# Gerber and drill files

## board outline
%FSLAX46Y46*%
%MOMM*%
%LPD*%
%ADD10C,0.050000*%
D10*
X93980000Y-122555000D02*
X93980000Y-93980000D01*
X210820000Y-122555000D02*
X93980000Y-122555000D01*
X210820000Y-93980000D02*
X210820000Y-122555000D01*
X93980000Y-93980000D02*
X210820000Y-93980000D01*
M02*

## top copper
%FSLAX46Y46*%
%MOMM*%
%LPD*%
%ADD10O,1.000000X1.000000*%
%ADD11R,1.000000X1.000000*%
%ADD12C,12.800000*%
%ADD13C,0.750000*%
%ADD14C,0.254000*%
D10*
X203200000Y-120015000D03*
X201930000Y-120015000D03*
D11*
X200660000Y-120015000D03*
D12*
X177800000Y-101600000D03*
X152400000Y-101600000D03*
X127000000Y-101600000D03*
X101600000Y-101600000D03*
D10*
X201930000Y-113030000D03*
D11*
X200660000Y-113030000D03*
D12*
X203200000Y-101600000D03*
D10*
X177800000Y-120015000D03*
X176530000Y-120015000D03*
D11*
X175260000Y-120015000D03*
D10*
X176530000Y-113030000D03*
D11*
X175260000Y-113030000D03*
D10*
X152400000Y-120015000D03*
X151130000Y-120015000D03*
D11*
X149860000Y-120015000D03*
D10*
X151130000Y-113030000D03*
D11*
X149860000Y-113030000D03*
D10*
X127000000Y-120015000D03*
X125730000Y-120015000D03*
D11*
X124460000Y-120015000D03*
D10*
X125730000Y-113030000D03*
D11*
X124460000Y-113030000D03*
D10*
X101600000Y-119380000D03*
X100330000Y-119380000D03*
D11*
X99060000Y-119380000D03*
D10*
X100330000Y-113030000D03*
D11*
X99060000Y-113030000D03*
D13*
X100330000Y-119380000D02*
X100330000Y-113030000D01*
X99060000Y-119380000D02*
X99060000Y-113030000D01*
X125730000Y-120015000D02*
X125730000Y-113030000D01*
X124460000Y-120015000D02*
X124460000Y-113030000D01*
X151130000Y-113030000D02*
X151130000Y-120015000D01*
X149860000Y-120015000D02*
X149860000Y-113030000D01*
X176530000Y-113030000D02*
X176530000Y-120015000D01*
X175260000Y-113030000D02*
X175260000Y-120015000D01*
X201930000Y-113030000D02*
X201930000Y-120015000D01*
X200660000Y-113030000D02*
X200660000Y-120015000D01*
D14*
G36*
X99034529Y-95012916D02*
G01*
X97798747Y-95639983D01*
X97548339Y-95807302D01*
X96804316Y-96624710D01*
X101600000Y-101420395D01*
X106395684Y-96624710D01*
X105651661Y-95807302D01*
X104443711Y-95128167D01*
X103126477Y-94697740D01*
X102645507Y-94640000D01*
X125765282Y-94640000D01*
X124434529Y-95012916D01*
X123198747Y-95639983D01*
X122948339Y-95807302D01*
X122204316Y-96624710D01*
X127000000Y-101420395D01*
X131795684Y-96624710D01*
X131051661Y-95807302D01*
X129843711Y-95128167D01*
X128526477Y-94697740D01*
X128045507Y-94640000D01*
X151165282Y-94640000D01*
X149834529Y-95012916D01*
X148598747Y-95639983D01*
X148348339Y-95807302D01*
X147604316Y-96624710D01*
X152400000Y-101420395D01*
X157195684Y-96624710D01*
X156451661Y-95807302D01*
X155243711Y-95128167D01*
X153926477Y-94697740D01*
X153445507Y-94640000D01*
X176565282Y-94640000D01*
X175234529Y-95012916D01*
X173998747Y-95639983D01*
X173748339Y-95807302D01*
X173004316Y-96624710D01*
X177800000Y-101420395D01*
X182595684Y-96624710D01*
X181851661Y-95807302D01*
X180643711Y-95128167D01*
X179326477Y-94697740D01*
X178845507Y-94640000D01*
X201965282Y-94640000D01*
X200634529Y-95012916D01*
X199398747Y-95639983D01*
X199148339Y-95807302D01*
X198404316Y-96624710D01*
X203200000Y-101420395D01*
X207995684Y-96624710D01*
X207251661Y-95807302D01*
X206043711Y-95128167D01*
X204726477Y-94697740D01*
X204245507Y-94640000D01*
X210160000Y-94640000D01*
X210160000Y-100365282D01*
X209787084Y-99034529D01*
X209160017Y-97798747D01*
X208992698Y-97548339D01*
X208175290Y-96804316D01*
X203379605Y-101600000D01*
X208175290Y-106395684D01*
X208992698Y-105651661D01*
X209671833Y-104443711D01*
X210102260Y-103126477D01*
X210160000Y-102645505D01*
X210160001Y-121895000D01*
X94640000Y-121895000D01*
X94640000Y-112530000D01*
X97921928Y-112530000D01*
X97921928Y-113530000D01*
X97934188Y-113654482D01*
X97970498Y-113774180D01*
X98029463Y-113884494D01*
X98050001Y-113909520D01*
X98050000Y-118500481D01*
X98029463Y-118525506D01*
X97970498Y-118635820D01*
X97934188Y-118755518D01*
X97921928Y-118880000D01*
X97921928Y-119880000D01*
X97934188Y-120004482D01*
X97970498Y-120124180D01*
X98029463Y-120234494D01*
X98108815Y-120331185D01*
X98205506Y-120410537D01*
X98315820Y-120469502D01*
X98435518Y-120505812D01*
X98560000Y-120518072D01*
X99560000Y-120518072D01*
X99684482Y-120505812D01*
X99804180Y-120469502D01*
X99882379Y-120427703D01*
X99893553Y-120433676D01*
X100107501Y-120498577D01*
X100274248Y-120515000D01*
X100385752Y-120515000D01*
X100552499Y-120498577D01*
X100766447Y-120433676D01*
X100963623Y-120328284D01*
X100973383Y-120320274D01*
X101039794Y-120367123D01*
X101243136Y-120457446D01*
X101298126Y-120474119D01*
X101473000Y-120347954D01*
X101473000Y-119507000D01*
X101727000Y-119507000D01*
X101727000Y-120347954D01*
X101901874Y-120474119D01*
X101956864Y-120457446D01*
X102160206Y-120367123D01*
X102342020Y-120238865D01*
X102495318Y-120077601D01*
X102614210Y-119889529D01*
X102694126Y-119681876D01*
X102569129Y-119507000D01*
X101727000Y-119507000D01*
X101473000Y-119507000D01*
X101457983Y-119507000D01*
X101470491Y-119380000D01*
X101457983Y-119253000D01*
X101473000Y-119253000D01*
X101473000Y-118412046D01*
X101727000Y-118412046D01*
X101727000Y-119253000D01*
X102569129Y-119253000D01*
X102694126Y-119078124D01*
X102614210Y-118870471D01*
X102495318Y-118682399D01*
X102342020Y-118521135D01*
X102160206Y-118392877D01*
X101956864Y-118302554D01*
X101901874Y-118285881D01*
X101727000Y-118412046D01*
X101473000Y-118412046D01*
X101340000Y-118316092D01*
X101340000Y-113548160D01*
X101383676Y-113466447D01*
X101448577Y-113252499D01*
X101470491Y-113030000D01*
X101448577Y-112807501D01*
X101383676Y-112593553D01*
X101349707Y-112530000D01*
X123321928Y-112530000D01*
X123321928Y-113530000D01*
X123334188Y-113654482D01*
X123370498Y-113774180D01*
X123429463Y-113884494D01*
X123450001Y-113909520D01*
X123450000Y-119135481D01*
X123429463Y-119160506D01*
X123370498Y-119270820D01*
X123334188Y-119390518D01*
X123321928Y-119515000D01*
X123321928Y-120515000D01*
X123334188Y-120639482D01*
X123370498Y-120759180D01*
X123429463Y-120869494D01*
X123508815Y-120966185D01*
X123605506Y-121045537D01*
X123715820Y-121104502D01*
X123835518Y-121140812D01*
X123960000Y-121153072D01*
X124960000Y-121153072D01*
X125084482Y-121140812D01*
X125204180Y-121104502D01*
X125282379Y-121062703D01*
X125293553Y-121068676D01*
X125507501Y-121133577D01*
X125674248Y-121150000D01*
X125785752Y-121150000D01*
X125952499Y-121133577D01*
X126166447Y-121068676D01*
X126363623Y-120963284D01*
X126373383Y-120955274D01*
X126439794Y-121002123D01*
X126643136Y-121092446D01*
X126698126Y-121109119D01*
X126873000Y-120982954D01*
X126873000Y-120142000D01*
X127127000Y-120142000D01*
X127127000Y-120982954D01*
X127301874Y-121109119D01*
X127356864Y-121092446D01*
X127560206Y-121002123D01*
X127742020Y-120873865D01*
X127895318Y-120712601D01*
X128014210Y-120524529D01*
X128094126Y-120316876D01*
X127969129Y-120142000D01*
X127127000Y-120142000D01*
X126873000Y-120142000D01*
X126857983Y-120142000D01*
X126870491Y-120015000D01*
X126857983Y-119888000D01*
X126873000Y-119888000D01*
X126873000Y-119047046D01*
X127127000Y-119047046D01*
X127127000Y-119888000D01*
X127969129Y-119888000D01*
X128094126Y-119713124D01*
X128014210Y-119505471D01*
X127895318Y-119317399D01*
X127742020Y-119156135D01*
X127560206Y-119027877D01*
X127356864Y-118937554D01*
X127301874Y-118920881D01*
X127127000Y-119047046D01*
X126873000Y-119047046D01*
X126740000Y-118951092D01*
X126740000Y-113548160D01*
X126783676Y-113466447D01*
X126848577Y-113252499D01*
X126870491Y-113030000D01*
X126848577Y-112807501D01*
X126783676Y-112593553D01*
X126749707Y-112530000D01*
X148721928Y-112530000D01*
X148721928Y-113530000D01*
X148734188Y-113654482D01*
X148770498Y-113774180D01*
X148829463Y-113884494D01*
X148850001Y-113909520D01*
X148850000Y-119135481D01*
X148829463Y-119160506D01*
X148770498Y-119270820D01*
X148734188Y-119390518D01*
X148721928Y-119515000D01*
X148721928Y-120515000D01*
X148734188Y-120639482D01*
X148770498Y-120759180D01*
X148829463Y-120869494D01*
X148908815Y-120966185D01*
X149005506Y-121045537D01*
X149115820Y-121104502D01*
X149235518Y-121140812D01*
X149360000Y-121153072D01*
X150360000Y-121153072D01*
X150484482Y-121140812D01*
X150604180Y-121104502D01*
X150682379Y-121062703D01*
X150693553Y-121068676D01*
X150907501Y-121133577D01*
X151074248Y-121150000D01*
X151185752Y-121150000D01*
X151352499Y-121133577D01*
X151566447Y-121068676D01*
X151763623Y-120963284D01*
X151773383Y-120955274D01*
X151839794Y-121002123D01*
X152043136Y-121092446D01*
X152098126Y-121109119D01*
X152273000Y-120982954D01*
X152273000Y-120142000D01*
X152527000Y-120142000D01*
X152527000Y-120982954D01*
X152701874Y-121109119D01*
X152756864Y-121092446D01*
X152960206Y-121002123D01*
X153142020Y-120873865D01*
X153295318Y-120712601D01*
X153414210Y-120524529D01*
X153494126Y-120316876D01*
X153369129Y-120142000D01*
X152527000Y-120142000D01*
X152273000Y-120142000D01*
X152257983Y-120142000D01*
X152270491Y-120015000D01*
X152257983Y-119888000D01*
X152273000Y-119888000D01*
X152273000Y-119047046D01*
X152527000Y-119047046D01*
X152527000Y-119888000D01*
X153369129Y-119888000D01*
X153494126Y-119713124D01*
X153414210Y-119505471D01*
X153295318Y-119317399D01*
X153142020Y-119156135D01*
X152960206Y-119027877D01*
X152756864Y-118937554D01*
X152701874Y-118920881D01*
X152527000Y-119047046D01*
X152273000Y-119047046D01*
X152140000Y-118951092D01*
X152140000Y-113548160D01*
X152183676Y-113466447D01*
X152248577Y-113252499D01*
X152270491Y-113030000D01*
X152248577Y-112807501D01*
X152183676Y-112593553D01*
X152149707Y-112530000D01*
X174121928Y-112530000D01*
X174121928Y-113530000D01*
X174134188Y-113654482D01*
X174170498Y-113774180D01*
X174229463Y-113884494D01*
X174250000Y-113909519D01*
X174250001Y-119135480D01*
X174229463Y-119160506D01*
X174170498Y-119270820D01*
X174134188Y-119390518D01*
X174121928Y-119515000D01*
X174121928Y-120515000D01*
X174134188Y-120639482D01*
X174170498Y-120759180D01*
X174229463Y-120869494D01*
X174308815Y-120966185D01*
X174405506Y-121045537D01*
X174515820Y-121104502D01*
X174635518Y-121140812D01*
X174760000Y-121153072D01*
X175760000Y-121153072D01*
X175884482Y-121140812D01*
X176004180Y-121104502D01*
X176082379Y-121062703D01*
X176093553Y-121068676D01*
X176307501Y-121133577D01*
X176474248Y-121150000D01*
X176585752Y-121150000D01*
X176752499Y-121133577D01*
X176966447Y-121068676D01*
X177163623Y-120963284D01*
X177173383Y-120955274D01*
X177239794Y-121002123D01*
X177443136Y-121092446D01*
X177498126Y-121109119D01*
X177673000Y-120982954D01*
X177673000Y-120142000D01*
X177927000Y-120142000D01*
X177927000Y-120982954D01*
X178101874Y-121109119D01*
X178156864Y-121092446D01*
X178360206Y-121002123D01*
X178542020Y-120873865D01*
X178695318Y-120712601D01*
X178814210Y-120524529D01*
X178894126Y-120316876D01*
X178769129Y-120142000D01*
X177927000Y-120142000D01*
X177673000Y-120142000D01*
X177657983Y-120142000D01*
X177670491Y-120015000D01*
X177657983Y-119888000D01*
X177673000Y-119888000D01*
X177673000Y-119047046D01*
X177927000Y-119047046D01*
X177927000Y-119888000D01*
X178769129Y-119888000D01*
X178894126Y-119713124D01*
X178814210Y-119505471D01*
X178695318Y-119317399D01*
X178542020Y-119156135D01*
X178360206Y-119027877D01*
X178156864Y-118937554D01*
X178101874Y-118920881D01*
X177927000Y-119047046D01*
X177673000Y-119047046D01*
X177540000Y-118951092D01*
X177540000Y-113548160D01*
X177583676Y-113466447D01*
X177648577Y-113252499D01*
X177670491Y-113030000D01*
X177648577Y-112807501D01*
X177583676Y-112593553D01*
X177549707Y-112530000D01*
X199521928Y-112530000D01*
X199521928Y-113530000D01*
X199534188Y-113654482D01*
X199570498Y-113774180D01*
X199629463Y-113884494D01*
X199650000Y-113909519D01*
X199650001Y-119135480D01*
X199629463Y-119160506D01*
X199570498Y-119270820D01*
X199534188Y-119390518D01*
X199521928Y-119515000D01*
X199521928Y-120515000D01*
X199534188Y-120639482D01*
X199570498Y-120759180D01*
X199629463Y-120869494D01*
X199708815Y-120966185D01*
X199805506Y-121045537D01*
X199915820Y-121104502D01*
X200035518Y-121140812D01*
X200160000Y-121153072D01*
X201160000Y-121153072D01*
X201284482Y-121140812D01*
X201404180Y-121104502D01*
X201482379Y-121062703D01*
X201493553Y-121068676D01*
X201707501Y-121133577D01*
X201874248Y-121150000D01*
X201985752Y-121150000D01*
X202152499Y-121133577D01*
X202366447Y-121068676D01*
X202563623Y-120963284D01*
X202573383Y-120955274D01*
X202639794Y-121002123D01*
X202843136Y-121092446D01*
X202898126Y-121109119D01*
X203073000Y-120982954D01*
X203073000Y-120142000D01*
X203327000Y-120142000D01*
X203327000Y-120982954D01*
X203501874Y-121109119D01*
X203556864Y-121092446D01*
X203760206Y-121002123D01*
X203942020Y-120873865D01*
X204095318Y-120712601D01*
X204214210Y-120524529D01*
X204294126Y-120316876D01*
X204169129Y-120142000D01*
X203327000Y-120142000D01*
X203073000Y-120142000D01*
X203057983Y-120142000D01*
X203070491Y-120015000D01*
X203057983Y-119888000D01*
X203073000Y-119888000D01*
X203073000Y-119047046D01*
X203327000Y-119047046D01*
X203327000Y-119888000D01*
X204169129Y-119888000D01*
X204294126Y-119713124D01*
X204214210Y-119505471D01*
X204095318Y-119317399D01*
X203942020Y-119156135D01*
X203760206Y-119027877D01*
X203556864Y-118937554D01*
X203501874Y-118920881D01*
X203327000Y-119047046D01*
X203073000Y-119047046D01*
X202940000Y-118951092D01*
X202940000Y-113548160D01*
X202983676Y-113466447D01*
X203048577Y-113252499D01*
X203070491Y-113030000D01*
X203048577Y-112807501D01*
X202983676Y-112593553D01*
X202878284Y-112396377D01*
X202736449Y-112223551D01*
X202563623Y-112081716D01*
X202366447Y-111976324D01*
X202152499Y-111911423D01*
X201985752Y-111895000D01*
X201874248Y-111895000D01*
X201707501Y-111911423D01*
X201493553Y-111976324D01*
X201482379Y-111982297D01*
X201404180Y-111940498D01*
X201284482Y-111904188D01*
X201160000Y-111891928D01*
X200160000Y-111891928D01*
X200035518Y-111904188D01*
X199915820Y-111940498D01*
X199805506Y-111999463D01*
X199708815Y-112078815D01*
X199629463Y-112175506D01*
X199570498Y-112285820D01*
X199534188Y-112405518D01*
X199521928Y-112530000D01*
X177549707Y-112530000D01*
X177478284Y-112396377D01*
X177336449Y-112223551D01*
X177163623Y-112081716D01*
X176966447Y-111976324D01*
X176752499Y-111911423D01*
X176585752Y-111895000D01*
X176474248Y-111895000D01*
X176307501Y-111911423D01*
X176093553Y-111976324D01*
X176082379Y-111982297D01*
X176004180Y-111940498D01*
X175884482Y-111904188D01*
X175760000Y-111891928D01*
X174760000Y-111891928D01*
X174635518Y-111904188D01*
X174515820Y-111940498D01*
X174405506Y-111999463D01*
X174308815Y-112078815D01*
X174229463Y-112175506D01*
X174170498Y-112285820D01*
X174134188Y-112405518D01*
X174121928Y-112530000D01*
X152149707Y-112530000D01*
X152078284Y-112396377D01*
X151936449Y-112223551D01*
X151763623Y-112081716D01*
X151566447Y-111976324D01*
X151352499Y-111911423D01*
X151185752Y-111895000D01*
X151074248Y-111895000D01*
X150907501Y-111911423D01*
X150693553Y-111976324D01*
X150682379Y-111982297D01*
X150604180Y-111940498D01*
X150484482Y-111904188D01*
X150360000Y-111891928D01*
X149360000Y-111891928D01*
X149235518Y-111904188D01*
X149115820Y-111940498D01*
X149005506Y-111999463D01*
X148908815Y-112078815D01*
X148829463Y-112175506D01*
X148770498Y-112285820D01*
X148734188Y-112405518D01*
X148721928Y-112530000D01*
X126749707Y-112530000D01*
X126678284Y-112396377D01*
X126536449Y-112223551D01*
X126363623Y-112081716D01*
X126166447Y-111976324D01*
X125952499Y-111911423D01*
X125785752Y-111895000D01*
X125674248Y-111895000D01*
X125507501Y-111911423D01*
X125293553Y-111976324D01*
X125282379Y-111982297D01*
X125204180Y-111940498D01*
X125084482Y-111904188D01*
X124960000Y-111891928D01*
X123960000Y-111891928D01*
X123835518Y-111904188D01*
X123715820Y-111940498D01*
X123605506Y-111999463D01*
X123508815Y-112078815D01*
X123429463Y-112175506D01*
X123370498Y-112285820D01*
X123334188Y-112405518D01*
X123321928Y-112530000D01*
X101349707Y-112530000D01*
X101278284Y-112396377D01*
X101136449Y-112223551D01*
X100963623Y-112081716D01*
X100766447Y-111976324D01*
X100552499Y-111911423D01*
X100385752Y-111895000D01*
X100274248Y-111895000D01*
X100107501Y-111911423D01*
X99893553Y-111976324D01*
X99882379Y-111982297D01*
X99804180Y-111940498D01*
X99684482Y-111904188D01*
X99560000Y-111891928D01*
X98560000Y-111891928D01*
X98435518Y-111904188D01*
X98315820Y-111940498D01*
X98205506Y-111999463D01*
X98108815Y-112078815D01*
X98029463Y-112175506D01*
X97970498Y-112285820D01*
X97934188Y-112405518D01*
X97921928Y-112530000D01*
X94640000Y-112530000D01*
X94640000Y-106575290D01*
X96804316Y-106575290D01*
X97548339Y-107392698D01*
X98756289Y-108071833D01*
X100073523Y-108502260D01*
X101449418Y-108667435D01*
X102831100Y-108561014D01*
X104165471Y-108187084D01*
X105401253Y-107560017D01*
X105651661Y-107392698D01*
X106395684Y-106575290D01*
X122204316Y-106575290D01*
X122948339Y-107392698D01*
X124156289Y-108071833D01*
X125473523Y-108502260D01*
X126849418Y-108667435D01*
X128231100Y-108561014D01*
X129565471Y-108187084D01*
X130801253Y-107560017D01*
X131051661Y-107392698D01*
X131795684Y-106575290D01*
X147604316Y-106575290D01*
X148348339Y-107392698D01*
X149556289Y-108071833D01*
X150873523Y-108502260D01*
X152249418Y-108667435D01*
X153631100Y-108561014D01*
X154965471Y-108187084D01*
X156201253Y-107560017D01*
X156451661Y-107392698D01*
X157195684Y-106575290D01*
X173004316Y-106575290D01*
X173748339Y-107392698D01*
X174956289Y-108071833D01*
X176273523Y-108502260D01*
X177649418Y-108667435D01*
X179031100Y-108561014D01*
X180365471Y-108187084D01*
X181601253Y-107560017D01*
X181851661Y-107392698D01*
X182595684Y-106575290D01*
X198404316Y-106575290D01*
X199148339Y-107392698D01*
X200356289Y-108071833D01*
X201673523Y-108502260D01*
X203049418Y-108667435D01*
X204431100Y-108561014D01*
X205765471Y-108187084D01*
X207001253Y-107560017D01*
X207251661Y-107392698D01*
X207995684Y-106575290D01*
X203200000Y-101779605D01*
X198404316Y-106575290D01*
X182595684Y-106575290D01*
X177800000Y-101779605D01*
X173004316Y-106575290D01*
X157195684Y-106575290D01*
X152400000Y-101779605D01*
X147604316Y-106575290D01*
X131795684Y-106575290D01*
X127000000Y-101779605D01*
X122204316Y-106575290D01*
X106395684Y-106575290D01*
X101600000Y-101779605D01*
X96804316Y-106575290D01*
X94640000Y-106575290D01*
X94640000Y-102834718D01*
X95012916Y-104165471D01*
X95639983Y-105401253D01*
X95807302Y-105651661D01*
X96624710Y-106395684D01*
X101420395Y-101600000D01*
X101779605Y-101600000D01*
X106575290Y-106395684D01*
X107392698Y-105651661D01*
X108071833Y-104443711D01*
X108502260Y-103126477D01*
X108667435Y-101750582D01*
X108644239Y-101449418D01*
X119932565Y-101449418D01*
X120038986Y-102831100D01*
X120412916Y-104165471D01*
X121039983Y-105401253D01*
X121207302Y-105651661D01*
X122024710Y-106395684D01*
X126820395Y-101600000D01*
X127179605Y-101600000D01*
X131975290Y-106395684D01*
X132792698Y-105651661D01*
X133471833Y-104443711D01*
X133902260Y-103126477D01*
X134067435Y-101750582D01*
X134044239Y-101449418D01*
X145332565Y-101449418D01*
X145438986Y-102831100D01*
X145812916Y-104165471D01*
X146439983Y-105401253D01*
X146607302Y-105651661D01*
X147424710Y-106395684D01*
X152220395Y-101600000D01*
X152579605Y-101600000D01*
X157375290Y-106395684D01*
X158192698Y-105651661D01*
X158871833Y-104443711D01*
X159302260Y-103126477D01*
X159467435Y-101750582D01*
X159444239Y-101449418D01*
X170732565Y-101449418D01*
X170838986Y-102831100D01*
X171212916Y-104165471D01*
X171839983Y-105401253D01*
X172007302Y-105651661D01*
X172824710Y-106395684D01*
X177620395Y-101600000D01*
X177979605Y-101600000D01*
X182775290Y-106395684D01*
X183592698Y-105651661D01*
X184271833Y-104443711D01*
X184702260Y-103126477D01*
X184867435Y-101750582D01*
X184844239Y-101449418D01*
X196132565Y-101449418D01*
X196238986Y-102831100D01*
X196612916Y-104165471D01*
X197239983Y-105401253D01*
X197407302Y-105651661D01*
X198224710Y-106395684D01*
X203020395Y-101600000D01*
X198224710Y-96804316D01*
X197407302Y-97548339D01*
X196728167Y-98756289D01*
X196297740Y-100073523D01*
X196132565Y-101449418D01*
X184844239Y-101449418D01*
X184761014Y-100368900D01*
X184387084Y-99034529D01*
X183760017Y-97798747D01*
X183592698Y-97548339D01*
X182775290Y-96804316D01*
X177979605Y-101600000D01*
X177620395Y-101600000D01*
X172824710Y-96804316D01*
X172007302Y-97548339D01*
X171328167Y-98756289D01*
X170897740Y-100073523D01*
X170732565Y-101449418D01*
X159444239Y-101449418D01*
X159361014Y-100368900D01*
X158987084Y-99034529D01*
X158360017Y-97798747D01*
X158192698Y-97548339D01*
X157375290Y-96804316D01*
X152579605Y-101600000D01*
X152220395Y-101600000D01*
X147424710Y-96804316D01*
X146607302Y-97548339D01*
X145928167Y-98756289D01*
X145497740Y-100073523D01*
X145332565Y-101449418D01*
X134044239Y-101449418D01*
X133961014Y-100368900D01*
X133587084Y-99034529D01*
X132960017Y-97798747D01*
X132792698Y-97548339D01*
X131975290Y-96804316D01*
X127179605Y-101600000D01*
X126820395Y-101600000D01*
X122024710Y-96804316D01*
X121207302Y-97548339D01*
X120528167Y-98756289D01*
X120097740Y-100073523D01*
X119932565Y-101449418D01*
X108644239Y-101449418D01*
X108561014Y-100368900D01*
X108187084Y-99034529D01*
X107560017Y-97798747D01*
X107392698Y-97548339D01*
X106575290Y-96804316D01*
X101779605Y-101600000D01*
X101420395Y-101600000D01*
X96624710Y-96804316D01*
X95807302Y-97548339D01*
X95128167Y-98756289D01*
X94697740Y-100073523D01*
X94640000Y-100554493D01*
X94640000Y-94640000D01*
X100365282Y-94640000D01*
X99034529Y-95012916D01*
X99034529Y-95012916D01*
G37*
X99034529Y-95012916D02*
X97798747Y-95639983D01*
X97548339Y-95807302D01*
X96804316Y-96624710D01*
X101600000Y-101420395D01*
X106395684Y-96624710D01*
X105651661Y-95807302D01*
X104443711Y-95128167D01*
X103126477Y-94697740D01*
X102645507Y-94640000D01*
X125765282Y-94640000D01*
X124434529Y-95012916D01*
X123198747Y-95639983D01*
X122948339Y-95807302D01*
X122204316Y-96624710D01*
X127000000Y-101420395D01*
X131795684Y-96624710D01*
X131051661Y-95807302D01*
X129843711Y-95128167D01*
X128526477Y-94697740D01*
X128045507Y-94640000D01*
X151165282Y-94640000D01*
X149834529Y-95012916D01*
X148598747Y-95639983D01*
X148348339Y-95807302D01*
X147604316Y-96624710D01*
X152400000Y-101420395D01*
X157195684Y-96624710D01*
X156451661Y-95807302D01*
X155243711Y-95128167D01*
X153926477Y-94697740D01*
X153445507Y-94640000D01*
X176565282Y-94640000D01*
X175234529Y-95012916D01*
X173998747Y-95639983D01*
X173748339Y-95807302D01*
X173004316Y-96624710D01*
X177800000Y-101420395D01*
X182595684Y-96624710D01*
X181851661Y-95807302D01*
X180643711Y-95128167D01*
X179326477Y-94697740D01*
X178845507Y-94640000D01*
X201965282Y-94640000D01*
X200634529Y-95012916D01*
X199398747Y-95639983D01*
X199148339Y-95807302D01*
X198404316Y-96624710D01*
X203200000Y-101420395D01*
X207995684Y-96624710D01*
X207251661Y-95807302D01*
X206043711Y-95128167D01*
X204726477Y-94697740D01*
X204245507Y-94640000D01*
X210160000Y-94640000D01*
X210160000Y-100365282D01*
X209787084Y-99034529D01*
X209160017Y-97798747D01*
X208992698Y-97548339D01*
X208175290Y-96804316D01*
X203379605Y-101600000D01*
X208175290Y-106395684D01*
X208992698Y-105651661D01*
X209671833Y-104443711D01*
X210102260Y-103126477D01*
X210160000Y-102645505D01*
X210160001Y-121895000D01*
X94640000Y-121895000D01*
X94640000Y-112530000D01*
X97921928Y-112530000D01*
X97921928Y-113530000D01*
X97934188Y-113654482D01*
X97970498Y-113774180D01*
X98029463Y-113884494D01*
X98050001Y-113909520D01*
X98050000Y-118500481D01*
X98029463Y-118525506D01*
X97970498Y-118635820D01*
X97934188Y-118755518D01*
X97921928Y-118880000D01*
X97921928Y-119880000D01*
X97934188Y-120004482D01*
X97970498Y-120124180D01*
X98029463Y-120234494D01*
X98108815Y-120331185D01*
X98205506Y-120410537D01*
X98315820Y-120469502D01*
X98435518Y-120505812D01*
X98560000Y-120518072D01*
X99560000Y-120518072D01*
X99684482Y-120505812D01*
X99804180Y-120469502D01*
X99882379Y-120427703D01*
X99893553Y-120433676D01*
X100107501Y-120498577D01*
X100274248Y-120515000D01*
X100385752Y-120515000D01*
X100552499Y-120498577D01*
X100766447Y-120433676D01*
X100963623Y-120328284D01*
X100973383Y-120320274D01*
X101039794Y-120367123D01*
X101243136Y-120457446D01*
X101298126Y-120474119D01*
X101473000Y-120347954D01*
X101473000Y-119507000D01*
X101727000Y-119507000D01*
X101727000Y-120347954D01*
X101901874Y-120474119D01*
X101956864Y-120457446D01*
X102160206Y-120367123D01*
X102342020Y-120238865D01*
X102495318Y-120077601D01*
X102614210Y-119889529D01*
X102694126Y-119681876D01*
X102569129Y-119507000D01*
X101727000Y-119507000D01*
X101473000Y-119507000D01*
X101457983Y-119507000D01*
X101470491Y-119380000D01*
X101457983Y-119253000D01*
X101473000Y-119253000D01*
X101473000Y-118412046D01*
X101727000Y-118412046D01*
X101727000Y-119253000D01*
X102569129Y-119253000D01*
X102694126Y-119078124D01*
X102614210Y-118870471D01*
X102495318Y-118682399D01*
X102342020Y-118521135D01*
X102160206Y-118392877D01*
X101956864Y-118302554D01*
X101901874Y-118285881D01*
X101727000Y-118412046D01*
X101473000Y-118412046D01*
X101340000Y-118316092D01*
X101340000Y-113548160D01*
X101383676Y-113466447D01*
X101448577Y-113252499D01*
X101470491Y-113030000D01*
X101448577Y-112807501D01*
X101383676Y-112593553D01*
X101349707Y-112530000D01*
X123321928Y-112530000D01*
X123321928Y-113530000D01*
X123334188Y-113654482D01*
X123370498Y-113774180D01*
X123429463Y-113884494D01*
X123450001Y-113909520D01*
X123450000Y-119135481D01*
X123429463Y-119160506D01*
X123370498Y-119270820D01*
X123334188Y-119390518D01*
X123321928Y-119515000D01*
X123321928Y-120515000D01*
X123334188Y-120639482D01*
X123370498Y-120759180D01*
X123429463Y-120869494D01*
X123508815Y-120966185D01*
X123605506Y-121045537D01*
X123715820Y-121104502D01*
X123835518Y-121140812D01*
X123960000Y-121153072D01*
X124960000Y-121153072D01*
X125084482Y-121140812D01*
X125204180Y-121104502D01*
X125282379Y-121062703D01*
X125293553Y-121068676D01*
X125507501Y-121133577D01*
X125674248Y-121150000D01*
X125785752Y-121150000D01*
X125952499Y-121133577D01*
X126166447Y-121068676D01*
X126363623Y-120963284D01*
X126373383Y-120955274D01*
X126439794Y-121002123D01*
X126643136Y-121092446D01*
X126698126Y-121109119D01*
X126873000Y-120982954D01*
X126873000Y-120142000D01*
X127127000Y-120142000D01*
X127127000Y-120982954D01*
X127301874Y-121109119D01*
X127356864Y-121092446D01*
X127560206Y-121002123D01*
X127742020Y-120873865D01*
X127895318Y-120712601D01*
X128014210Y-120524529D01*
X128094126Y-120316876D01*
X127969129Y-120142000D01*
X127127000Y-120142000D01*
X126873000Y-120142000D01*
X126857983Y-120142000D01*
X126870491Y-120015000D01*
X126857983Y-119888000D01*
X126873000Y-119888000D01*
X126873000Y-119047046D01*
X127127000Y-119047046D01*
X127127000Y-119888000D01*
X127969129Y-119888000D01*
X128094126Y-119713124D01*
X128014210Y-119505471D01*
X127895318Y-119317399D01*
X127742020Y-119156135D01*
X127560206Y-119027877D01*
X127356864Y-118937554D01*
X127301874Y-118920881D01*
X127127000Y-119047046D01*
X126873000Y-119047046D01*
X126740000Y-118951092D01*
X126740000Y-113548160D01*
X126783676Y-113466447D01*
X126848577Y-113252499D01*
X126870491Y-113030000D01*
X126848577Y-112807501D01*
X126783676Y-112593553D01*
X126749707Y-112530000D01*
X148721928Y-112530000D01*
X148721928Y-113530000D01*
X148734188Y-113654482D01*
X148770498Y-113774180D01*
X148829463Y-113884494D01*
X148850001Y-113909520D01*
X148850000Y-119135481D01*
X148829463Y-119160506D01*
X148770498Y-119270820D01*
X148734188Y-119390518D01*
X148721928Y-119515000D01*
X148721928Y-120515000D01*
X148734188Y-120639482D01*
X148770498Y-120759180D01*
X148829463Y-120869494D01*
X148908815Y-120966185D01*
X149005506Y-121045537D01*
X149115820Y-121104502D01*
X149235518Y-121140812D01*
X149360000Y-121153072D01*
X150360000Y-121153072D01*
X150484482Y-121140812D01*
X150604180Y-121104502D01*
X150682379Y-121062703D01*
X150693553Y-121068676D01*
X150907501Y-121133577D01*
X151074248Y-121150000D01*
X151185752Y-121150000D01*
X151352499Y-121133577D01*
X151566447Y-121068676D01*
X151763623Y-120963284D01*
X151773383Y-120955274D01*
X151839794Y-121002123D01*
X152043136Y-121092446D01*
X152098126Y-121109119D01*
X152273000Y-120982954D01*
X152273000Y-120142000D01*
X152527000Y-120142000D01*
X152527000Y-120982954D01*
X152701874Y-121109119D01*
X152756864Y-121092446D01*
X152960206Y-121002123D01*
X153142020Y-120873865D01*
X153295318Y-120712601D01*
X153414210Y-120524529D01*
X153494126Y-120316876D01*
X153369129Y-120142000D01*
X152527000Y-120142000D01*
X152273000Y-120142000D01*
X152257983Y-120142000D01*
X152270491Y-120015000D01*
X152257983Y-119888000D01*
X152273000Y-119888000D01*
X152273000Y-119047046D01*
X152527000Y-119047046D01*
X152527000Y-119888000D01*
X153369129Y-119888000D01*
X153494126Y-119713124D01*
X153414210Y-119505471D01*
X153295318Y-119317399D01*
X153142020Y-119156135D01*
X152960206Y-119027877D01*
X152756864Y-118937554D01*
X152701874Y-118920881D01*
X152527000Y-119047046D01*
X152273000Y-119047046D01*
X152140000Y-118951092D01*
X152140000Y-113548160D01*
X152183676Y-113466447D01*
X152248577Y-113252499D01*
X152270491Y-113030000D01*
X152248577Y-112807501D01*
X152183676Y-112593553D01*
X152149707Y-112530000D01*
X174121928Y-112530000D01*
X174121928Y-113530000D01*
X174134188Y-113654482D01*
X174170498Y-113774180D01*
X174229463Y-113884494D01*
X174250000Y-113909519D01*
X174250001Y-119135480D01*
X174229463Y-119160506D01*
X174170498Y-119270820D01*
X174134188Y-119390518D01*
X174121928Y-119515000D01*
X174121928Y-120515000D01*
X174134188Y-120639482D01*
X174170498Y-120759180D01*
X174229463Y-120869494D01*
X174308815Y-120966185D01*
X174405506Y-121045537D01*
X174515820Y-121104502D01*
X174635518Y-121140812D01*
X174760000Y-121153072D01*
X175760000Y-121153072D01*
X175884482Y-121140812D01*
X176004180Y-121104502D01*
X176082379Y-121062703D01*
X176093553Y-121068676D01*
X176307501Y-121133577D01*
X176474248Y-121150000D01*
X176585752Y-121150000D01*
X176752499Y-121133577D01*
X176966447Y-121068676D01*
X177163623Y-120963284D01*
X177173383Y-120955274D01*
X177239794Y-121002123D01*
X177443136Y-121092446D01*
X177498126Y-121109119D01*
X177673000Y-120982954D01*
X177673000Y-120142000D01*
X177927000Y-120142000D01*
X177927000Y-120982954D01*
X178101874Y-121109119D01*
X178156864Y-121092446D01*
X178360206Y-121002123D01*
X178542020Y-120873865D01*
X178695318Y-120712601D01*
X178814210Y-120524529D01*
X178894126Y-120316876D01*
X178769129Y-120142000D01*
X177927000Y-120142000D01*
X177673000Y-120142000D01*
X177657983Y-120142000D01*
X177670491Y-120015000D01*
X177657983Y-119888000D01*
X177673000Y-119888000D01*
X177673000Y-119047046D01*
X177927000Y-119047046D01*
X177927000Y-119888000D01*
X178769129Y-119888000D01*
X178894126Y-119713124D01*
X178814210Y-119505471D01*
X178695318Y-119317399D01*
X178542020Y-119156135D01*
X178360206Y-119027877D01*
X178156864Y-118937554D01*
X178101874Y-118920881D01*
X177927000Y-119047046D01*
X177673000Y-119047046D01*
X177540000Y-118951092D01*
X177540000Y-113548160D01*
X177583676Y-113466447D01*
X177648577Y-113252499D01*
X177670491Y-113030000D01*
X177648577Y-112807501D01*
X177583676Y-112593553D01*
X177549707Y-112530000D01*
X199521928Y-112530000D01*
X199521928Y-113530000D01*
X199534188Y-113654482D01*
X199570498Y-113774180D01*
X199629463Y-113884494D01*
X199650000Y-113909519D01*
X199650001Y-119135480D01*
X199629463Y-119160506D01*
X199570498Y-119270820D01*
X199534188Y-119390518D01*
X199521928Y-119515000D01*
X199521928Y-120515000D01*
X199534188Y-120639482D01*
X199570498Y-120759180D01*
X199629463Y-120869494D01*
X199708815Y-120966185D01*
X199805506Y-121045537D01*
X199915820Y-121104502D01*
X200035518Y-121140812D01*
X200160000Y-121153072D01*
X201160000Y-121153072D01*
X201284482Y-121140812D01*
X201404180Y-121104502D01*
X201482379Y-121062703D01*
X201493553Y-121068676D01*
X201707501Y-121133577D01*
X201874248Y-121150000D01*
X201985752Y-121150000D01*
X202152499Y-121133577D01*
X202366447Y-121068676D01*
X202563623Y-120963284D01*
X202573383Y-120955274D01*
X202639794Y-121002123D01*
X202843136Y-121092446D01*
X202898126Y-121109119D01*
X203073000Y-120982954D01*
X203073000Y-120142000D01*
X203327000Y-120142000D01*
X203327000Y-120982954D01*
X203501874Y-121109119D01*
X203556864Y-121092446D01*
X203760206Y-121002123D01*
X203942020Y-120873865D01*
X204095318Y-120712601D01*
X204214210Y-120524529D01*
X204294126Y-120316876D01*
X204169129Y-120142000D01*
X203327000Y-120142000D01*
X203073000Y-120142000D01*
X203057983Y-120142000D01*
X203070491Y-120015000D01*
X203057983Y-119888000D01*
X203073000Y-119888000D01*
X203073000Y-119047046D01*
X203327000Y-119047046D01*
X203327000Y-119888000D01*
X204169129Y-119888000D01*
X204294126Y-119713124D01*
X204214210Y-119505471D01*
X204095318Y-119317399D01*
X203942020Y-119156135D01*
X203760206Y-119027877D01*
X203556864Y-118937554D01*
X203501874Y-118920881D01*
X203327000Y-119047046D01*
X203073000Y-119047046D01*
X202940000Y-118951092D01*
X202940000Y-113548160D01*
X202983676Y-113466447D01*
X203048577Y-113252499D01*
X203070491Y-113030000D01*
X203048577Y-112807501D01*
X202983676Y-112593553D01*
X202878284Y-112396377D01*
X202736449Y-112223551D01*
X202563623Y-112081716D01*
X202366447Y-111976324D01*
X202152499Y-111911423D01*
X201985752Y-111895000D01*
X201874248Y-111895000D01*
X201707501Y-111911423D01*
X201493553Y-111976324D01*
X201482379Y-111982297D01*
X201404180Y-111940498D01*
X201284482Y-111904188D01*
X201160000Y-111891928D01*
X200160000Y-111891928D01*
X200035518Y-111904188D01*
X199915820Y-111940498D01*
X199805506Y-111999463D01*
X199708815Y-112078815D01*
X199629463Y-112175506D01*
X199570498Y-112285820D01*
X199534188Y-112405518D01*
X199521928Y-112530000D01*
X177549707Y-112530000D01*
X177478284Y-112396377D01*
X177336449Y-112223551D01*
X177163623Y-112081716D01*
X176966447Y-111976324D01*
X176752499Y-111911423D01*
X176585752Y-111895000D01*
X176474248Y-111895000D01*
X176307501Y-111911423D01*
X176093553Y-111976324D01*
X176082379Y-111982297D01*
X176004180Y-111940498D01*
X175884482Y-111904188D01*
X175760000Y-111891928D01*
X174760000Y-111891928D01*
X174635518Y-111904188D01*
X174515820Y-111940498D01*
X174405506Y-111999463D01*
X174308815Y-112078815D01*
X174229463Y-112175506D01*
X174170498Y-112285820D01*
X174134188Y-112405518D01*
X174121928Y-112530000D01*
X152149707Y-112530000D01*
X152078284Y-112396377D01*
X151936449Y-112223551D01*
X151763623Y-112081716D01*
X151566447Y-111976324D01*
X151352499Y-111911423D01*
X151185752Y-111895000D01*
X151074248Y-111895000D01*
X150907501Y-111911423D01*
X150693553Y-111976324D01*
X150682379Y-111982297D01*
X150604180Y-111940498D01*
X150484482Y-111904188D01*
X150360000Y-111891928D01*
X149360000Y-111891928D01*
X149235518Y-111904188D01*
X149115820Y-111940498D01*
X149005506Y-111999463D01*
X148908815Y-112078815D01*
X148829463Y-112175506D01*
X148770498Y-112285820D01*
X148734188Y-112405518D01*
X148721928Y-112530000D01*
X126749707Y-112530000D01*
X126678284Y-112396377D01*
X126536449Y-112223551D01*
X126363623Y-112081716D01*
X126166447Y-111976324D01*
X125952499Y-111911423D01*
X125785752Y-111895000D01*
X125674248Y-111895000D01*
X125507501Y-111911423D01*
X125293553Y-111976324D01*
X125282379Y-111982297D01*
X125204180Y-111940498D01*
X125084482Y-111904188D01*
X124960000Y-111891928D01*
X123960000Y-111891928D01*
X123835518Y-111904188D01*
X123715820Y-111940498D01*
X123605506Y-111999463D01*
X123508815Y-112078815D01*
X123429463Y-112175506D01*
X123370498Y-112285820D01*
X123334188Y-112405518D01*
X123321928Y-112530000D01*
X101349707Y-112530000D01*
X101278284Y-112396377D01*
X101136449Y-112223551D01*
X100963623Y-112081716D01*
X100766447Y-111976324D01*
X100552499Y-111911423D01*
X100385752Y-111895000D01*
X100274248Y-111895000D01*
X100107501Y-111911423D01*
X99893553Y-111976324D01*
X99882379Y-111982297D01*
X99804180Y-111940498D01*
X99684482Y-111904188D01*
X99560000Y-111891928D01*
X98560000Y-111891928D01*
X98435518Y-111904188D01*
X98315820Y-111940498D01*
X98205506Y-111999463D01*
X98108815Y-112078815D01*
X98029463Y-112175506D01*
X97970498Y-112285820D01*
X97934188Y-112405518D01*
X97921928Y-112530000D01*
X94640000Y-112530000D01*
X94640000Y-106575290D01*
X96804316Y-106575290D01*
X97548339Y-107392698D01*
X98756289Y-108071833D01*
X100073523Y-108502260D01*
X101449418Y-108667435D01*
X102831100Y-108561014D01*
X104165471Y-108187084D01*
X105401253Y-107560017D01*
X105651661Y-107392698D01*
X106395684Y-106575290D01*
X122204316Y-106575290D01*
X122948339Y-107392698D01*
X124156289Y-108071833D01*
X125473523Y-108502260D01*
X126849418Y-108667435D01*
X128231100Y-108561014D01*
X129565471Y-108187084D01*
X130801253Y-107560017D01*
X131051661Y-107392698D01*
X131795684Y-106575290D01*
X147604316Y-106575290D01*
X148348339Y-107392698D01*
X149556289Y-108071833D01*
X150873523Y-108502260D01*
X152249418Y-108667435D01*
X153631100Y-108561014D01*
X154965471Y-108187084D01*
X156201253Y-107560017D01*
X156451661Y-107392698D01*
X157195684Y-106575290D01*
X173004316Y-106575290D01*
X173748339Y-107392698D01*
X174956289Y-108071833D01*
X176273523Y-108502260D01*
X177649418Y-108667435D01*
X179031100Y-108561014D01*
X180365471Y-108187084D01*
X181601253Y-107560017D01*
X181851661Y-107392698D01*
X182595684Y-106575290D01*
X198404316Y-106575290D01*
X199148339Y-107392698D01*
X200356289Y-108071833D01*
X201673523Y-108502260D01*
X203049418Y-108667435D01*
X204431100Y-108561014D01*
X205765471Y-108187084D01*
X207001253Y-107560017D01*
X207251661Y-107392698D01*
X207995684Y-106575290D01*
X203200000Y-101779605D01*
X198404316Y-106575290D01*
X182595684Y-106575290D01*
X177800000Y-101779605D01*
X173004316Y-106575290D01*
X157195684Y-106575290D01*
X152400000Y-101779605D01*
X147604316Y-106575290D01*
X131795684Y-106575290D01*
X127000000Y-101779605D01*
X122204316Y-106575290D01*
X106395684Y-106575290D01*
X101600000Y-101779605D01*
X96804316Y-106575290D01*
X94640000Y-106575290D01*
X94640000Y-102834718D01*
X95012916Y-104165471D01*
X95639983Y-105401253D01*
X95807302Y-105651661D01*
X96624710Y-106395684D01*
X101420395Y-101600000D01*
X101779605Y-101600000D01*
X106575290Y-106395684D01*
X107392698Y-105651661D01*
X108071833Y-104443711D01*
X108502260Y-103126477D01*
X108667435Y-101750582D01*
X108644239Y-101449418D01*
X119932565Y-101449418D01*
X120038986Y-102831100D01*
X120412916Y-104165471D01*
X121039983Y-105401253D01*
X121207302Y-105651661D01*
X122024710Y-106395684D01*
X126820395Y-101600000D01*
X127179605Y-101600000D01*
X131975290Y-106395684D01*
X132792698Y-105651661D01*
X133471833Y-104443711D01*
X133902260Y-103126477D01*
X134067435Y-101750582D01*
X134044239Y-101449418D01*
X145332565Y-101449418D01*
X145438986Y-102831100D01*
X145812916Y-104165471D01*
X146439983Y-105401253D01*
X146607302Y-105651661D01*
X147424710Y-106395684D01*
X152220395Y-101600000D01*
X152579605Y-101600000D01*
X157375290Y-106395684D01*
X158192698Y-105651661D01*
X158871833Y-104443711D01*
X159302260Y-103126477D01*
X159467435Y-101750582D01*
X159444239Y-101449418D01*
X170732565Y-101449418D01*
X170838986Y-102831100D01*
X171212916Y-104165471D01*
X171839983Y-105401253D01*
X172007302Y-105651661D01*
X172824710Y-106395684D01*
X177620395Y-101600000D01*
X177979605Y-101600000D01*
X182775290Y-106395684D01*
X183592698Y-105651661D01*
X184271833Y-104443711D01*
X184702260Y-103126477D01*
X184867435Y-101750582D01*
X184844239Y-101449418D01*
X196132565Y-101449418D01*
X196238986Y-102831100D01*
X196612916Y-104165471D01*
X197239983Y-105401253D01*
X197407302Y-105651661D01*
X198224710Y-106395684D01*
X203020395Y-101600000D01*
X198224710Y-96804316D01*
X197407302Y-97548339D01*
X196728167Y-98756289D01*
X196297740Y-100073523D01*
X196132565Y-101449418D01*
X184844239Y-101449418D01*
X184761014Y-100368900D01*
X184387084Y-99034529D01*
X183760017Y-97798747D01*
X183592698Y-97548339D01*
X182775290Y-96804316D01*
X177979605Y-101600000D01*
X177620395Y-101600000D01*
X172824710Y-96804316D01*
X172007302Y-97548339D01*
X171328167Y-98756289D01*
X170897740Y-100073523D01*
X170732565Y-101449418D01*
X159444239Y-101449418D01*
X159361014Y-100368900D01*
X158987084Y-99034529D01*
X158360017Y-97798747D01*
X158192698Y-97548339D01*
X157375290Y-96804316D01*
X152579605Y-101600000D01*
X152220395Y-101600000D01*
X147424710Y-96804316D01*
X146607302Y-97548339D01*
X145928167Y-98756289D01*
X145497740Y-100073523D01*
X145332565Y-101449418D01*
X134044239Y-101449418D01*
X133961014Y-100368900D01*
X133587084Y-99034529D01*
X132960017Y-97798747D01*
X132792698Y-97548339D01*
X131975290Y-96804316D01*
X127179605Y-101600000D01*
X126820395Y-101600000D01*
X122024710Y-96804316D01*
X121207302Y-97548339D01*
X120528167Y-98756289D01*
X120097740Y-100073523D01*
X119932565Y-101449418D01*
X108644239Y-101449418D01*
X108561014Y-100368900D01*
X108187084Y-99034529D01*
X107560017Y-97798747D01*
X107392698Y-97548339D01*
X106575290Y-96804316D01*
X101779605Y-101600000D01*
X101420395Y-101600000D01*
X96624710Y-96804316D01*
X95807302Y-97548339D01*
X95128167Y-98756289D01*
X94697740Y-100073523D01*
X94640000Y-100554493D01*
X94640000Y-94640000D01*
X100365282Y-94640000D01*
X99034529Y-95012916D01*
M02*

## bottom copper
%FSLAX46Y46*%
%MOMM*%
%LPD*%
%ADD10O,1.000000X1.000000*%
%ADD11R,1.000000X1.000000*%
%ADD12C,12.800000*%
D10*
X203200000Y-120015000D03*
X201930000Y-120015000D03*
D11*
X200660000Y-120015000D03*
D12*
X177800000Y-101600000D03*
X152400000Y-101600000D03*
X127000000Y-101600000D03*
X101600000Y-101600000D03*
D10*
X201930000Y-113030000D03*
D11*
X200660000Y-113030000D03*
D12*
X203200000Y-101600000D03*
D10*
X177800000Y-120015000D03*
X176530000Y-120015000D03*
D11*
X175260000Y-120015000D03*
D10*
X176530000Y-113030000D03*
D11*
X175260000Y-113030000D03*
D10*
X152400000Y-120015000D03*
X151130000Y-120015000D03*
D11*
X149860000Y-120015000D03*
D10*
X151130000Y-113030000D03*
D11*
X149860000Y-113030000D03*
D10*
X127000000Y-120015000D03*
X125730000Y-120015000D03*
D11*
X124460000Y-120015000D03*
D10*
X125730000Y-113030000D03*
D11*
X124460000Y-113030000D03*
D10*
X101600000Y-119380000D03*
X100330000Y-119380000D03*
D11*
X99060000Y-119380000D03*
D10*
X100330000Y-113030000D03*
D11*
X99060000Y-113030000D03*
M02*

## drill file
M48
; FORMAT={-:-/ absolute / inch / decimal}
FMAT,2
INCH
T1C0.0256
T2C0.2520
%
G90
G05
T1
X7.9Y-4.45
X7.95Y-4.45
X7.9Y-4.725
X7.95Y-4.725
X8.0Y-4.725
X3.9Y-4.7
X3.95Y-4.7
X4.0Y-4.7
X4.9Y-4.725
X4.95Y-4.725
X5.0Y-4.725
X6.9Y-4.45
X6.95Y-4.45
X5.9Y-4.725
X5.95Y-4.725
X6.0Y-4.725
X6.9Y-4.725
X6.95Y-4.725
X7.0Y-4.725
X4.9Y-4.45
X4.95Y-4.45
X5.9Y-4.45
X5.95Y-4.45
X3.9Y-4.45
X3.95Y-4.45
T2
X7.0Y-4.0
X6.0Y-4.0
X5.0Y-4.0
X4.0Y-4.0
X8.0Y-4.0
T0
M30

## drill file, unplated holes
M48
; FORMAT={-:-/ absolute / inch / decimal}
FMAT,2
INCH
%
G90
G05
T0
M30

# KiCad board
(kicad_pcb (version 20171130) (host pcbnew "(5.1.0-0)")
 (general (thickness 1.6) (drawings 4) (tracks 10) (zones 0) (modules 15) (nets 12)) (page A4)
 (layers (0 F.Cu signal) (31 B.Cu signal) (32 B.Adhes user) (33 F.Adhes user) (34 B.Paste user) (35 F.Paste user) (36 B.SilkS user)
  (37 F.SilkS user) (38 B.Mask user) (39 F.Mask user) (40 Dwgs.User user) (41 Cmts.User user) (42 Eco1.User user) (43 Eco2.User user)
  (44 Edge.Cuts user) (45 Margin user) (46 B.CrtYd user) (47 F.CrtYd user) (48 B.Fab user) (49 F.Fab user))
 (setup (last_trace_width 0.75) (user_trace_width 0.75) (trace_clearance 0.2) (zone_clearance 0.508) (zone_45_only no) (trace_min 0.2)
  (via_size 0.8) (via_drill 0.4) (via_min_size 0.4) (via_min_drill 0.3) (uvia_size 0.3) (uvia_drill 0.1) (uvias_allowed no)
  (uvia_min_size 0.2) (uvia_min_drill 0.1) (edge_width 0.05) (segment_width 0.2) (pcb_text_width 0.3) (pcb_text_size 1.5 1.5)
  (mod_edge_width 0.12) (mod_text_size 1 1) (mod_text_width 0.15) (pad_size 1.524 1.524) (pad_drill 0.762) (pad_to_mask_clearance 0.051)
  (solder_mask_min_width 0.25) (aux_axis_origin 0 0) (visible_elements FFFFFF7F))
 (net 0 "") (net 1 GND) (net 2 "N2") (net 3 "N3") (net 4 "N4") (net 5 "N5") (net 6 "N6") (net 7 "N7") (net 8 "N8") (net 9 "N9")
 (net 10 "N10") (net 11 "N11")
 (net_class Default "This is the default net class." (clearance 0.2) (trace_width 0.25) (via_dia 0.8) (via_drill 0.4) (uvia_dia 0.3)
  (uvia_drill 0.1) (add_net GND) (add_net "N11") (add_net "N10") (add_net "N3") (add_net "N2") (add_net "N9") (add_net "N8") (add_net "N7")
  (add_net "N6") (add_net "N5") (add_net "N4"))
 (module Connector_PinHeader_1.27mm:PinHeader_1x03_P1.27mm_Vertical (layer F.Cu) (at 200.66 120.015 90)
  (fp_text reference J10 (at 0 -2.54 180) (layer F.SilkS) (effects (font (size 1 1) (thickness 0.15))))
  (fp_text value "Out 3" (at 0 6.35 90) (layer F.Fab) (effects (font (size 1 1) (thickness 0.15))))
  (pad 3 thru_hole oval (at 0 2.54 90) (size 1 1) (drill 0.65) (layers *.Cu *.Mask) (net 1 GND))
  (pad 2 thru_hole oval (at 0 1.27 90) (size 1 1) (drill 0.65) (layers *.Cu *.Mask) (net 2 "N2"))
  (pad 1 thru_hole rect (at 0 0 90) (size 1 1) (drill 0.65) (layers *.Cu *.Mask) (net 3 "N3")))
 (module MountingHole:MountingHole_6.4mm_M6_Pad (layer F.Cu) (at 177.8 101.6)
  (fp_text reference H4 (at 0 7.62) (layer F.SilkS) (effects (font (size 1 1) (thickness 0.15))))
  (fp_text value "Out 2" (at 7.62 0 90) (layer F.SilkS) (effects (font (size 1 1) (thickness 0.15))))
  (pad 1 thru_hole circle (at 0 0) (size 12.8 12.8) (drill 6.4) (layers *.Cu *.Mask) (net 1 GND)))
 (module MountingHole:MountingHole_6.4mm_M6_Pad (layer F.Cu) (at 152.4 101.6)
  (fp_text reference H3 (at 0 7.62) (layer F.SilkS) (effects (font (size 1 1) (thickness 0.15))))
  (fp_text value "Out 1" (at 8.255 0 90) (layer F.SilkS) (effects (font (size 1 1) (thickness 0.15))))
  (pad 1 thru_hole circle (at 0 0) (size 12.8 12.8) (drill 6.4) (layers *.Cu *.Mask) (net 1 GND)))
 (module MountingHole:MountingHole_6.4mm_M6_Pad (layer F.Cu) (at 127 101.6)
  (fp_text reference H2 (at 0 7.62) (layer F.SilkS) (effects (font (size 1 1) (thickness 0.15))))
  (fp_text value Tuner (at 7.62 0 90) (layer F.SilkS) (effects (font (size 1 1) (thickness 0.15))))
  (pad 1 thru_hole circle (at 0 0) (size 12.8 12.8) (drill 6.4) (layers *.Cu *.Mask) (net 1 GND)))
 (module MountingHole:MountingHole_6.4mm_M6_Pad (layer F.Cu) (at 101.6 101.6)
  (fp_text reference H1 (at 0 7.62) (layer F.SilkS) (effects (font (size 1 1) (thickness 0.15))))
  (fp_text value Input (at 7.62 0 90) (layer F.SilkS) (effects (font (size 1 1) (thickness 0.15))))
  (pad 1 thru_hole circle (at 0 0) (size 12.8 12.8) (drill 6.4) (layers *.Cu *.Mask) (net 1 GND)))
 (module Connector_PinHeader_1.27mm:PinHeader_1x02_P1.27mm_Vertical (layer F.Cu) (at 200.66 113.03 90)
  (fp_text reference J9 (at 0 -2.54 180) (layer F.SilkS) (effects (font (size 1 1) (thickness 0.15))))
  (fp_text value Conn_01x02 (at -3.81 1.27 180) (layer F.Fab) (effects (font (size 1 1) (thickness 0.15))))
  (pad 2 thru_hole oval (at 0 1.27 90) (size 1 1) (drill 0.65) (layers *.Cu *.Mask) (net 2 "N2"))
  (pad 1 thru_hole rect (at 0 0 90) (size 1 1) (drill 0.65) (layers *.Cu *.Mask) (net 3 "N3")))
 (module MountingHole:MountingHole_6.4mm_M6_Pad (layer F.Cu) (at 203.2 101.6)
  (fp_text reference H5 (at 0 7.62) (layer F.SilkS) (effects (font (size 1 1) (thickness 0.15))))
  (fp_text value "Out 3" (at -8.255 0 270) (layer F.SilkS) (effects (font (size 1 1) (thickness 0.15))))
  (pad 1 thru_hole circle (at 0 0) (size 12.8 12.8) (drill 6.4) (layers *.Cu *.Mask) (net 1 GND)))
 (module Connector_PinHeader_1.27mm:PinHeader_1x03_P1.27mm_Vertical (layer F.Cu) (at 175.26 120.015 90)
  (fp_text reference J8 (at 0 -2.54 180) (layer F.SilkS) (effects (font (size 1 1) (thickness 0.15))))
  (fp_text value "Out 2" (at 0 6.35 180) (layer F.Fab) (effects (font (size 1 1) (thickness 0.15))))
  (pad 3 thru_hole oval (at 0 2.54 90) (size 1 1) (drill 0.65) (layers *.Cu *.Mask) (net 1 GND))
  (pad 2 thru_hole oval (at 0 1.27 90) (size 1 1) (drill 0.65) (layers *.Cu *.Mask) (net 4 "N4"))
  (pad 1 thru_hole rect (at 0 0 90) (size 1 1) (drill 0.65) (layers *.Cu *.Mask) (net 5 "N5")))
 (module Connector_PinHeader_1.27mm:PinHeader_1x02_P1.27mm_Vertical (layer F.Cu) (at 175.26 113.03 90)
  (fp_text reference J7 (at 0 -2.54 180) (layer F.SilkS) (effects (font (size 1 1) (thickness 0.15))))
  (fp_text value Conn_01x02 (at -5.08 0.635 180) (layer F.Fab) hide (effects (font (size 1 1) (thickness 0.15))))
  (pad 2 thru_hole oval (at 0 1.27 90) (size 1 1) (drill 0.65) (layers *.Cu *.Mask) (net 4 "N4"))
  (pad 1 thru_hole rect (at 0 0 90) (size 1 1) (drill 0.65) (layers *.Cu *.Mask) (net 5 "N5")))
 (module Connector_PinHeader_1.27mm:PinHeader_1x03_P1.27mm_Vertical (layer F.Cu) (at 149.86 120.015 90)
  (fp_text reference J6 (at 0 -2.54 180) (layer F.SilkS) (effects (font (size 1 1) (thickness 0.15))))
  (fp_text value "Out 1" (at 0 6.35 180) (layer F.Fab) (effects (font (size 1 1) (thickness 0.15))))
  (pad 3 thru_hole oval (at 0 2.54 90) (size 1 1) (drill 0.65) (layers *.Cu *.Mask) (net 1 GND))
  (pad 2 thru_hole oval (at 0 1.27 90) (size 1 1) (drill 0.65) (layers *.Cu *.Mask) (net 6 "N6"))
  (pad 1 thru_hole rect (at 0 0 90) (size 1 1) (drill 0.65) (layers *.Cu *.Mask) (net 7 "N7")))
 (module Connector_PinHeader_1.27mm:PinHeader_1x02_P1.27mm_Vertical (layer F.Cu) (at 149.86 113.03 90)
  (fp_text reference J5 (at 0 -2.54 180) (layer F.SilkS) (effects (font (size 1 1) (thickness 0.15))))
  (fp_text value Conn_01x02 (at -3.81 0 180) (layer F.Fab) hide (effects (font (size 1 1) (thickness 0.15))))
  (pad 2 thru_hole oval (at 0 1.27 90) (size 1 1) (drill 0.65) (layers *.Cu *.Mask) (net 6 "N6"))
  (pad 1 thru_hole rect (at 0 0 90) (size 1 1) (drill 0.65) (layers *.Cu *.Mask) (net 7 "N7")))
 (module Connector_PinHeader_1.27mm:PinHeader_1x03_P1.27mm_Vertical (layer F.Cu) (at 124.46 120.015 90)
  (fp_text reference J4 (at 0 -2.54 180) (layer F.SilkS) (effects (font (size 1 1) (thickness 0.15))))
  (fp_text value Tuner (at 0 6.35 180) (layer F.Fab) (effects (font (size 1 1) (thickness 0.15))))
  (pad 3 thru_hole oval (at 0 2.54 90) (size 1 1) (drill 0.65) (layers *.Cu *.Mask) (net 1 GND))
  (pad 2 thru_hole oval (at 0 1.27 90) (size 1 1) (drill 0.65) (layers *.Cu *.Mask) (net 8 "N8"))
  (pad 1 thru_hole rect (at 0 0 90) (size 1 1) (drill 0.65) (layers *.Cu *.Mask) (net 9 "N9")))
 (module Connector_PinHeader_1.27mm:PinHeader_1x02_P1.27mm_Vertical (layer F.Cu) (at 124.46 113.03 90)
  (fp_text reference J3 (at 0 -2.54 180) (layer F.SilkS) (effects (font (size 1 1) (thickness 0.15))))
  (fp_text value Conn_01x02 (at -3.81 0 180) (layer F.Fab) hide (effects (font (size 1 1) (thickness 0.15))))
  (pad 2 thru_hole oval (at 0 1.27 90) (size 1 1) (drill 0.65) (layers *.Cu *.Mask) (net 8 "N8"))
  (pad 1 thru_hole rect (at 0 0 90) (size 1 1) (drill 0.65) (layers *.Cu *.Mask) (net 9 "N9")))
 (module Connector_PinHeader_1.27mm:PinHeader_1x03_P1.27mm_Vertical (layer F.Cu) (at 99.06 119.38 90)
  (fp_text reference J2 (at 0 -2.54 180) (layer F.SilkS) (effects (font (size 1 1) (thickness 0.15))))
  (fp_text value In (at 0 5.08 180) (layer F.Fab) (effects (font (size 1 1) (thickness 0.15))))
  (pad 3 thru_hole oval (at 0 2.54 90) (size 1 1) (drill 0.65) (layers *.Cu *.Mask) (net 1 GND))
  (pad 2 thru_hole oval (at 0 1.27 90) (size 1 1) (drill 0.65) (layers *.Cu *.Mask) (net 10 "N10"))
  (pad 1 thru_hole rect (at 0 0 90) (size 1 1) (drill 0.65) (layers *.Cu *.Mask) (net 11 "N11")))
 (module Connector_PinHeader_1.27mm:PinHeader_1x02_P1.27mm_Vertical (layer F.Cu) (at 99.06 113.03 90)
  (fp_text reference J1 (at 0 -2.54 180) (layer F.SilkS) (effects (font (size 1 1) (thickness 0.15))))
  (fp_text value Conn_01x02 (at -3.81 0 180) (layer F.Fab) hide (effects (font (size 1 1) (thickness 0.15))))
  (pad 2 thru_hole oval (at 0 1.27 90) (size 1 1) (drill 0.65) (layers *.Cu *.Mask) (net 10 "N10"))
  (pad 1 thru_hole rect (at 0 0 90) (size 1 1) (drill 0.65) (layers *.Cu *.Mask) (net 11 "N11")))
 (gr_line (start 93.98 122.555) (end 93.98 93.98) (layer Edge.Cuts) (width 0.05))
 (gr_line (start 210.82 122.555) (end 93.98 122.555) (layer Edge.Cuts) (width 0.05))
 (gr_line (start 210.82 93.98) (end 210.82 122.555) (layer Edge.Cuts) (width 0.05))
 (gr_line (start 93.98 93.98) (end 210.82 93.98) (layer Edge.Cuts) (width 0.05))
 (segment (start 100.33 119.38) (end 100.33 113.03) (width 0.75) (layer F.Cu) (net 10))
 (segment (start 99.06 119.38) (end 99.06 113.03) (width 0.75) (layer F.Cu) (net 11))
 (segment (start 125.73 120.015) (end 125.73 113.03) (width 0.75) (layer F.Cu) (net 8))
 (segment (start 124.46 120.015) (end 124.46 113.03) (width 0.75) (layer F.Cu) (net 9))
 (segment (start 151.13 113.03) (end 151.13 120.015) (width 0.75) (layer F.Cu) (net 6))
 (segment (start 149.86 120.015) (end 149.86 113.03) (width 0.75) (layer F.Cu) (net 7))
 (segment (start 176.53 113.03) (end 176.53 120.015) (width 0.75) (layer F.Cu) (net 4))
 (segment (start 175.26 113.03) (end 175.26 120.015) (width 0.75) (layer F.Cu) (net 5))
 (segment (start 201.93 113.03) (end 201.93 120.015) (width 0.75) (layer F.Cu) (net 2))
 (segment (start 200.66 113.03) (end 200.66 120.015) (width 0.75) (layer F.Cu) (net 3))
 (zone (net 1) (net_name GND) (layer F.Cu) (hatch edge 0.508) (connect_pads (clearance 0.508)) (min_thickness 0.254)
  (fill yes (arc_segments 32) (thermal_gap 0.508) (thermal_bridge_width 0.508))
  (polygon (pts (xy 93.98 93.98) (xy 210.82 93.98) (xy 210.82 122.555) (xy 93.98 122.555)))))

